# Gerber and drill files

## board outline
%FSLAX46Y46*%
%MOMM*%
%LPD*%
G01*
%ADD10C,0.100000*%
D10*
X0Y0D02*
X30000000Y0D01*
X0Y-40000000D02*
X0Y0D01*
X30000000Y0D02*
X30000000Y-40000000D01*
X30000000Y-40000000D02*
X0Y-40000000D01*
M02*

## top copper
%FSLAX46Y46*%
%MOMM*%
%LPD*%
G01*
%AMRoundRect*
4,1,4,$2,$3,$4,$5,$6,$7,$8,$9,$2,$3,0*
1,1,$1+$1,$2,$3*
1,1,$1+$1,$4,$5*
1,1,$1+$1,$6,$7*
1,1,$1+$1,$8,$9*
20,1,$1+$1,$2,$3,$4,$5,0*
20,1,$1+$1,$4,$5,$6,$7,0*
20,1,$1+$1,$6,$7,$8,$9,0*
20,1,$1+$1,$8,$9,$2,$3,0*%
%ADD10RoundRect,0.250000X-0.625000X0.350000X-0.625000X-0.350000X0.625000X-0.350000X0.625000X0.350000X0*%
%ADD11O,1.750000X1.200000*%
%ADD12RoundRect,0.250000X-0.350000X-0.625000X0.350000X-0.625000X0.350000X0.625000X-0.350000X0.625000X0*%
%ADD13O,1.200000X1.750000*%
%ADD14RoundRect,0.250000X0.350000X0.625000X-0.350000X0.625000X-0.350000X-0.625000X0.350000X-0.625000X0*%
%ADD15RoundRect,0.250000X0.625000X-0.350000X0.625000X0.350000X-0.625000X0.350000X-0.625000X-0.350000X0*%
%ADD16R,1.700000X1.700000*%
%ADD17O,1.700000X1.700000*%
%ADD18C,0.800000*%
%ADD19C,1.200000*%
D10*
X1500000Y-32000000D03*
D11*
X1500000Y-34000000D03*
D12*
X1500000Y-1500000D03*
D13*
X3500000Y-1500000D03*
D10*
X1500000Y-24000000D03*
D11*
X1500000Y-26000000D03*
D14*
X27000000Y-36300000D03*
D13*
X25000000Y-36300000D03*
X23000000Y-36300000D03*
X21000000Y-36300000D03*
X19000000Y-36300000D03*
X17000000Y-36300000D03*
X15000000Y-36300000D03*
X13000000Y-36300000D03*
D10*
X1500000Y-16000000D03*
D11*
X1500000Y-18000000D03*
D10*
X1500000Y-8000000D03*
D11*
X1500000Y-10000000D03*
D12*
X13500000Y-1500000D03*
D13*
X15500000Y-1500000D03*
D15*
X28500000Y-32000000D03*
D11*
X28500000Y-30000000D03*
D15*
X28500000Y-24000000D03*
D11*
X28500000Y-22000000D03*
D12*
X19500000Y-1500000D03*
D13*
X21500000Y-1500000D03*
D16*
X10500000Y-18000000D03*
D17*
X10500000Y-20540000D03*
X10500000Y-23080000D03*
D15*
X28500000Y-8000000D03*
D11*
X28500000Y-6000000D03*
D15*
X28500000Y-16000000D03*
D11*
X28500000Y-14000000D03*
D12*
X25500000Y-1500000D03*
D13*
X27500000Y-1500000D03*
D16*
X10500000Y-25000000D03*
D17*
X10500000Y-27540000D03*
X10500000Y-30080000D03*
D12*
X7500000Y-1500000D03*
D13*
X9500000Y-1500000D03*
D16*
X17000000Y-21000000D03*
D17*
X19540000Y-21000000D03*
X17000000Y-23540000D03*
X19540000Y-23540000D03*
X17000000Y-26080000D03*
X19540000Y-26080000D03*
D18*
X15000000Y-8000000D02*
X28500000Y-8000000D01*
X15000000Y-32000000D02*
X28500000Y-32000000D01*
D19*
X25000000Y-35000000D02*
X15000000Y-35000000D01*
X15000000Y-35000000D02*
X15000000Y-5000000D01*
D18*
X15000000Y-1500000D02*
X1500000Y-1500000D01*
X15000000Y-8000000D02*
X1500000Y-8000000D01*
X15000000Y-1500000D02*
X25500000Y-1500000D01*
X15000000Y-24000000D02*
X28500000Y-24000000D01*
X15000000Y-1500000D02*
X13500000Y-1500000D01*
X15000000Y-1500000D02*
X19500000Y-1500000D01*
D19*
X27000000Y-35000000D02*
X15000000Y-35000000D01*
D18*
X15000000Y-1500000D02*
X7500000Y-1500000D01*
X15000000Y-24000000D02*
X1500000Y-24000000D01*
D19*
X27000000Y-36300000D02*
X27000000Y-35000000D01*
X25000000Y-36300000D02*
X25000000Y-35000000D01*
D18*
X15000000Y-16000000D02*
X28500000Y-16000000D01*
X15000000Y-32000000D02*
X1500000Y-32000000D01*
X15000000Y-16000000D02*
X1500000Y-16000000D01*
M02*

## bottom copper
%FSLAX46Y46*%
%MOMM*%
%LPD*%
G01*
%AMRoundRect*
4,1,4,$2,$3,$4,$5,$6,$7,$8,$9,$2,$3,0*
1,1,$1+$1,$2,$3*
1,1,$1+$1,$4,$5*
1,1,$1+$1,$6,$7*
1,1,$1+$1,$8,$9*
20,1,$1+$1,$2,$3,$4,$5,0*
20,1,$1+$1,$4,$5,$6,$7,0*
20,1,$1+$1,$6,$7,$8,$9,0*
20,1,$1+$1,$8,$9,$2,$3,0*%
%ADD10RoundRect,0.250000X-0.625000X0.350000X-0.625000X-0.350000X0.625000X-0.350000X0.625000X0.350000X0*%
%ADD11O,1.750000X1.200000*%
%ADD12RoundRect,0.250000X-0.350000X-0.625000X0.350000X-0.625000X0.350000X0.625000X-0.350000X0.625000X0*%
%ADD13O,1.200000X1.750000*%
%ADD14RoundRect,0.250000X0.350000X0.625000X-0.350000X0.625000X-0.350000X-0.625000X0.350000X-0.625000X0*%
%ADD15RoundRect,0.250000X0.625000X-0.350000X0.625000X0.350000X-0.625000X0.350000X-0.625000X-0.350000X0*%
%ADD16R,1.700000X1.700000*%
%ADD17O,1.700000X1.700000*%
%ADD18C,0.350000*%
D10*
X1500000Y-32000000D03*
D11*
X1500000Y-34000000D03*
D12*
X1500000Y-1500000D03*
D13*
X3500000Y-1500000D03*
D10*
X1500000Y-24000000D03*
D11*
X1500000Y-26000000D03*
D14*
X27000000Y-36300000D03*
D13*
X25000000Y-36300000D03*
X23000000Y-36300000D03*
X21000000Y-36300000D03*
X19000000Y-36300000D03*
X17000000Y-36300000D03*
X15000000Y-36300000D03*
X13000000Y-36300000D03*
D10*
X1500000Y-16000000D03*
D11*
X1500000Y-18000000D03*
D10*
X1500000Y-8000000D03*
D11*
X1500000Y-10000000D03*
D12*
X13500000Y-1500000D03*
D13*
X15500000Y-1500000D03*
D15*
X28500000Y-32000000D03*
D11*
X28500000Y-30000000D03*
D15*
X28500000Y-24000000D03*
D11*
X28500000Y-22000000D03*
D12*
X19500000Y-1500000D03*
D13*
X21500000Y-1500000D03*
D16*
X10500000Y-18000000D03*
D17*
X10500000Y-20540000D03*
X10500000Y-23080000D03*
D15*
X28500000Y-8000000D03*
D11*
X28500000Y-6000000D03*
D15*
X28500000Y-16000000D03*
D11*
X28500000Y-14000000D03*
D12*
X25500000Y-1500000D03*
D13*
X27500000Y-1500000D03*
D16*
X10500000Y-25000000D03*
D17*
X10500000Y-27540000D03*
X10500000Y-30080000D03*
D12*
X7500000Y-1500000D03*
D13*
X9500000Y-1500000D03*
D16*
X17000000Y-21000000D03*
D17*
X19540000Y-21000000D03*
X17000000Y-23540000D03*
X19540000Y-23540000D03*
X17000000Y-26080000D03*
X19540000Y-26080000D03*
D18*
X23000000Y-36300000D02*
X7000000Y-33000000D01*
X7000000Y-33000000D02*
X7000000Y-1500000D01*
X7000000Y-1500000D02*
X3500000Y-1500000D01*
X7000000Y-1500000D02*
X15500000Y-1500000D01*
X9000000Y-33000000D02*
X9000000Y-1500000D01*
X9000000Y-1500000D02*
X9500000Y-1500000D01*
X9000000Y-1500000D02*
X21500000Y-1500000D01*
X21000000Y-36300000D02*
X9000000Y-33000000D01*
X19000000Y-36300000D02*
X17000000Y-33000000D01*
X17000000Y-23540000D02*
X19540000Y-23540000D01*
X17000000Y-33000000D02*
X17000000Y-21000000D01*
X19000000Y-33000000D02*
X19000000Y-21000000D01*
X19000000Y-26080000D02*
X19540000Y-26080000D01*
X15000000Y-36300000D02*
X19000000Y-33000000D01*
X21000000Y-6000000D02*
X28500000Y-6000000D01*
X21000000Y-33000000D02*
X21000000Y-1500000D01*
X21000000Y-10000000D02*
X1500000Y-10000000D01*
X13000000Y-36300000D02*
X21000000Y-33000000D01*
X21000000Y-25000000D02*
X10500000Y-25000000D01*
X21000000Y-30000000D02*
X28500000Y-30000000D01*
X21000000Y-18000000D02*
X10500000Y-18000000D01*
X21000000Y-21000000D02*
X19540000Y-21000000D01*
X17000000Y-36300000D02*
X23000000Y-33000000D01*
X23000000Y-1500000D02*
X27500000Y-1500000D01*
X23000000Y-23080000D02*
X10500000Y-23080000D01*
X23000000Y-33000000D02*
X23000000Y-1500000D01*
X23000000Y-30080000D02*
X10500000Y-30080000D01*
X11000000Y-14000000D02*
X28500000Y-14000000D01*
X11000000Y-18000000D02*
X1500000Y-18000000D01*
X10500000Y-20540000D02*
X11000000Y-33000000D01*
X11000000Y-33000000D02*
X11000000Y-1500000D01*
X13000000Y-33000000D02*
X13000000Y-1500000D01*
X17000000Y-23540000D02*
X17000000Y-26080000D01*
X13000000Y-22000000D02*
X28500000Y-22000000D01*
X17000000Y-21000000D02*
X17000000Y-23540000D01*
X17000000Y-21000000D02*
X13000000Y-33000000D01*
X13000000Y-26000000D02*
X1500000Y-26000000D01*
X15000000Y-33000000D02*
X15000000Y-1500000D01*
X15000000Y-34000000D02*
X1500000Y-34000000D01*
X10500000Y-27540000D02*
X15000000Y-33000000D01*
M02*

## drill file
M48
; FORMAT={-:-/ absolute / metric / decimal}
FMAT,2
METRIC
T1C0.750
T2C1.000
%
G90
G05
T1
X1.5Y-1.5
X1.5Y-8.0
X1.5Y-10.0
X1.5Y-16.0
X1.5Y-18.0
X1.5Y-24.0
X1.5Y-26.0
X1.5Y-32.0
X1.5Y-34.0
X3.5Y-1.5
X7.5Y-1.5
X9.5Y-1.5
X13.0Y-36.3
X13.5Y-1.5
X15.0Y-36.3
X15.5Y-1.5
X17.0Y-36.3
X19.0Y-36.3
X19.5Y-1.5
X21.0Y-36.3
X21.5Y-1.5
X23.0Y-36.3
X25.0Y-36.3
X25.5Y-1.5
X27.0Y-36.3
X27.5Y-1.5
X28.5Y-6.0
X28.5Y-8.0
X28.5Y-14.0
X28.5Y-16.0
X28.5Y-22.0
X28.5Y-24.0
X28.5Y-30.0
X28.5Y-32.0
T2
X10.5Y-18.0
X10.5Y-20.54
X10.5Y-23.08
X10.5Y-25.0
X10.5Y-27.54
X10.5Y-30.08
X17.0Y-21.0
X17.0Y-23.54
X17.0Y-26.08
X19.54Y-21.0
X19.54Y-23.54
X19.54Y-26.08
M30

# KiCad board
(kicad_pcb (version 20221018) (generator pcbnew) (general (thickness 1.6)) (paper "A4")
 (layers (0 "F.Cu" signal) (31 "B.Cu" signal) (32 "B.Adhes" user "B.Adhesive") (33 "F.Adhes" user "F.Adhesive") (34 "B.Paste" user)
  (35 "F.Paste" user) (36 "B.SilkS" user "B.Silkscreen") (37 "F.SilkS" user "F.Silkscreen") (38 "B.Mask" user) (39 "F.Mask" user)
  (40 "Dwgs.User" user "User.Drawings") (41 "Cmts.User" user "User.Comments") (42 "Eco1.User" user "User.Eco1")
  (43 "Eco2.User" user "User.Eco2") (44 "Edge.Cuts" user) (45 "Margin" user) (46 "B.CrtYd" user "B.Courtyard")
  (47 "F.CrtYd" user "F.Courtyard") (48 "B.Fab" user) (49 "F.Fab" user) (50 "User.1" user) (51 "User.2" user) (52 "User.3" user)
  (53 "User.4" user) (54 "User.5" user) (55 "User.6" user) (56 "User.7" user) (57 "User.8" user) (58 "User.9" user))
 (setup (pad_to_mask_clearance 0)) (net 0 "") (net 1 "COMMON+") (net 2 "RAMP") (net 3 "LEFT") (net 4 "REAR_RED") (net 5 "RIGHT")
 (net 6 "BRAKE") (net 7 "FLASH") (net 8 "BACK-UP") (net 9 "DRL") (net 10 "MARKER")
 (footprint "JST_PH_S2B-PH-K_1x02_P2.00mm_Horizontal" (layer "F.Cu") (at 1.5 32 -90)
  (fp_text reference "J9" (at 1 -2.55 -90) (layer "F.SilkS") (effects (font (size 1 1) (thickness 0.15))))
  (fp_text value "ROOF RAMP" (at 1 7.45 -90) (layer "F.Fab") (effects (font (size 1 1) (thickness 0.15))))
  (pad "1" thru_hole roundrect (at 0 0 270) (size 1.2 1.75) (drill 0.75) (layers "*.Cu" "*.Mask") (roundrect_rratio 0.208333)
   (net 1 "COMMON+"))
  (pad "2" thru_hole oval (at 2 0 270) (size 1.2 1.75) (drill 0.75) (layers "*.Cu" "*.Mask") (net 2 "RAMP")))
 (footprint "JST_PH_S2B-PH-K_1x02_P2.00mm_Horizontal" (layer "F.Cu") (at 1.5 1.5)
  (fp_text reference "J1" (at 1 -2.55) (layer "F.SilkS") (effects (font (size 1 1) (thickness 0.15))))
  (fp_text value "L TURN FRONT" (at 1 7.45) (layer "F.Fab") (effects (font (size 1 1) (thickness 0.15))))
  (pad "1" thru_hole roundrect (at 0 0) (size 1.2 1.75) (drill 0.75) (layers "*.Cu" "*.Mask") (roundrect_rratio 0.208333) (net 1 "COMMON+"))
  (pad "2" thru_hole oval (at 2 0) (size 1.2 1.75) (drill 0.75) (layers "*.Cu" "*.Mask") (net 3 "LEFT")))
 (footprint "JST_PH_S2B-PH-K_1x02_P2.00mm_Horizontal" (layer "F.Cu") (at 1.5 24 -90)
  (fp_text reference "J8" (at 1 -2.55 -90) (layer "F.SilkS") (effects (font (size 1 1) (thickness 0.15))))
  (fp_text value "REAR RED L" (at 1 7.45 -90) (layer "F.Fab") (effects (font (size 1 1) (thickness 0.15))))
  (pad "1" thru_hole roundrect (at 0 0 270) (size 1.2 1.75) (drill 0.75) (layers "*.Cu" "*.Mask") (roundrect_rratio 0.208333)
   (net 1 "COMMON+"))
  (pad "2" thru_hole oval (at 2 0 270) (size 1.2 1.75) (drill 0.75) (layers "*.Cu" "*.Mask") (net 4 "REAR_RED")))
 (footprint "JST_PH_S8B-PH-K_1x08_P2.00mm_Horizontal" (layer "F.Cu") (at 27 36.3 180)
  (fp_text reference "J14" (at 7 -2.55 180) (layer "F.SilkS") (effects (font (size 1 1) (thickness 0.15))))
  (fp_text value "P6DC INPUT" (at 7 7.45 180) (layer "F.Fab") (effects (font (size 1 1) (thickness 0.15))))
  (pad "1" thru_hole roundrect (at 0 0 180) (size 1.2 1.75) (drill 0.75) (layers "*.Cu" "*.Mask") (roundrect_rratio 0.208333)
   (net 1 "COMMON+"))
  (pad "2" thru_hole oval (at 2 0 180) (size 1.2 1.75) (drill 0.75) (layers "*.Cu" "*.Mask") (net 1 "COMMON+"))
  (pad "3" thru_hole oval (at 4 0 180) (size 1.2 1.75) (drill 0.75) (layers "*.Cu" "*.Mask") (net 3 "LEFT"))
  (pad "4" thru_hole oval (at 6 0 180) (size 1.2 1.75) (drill 0.75) (layers "*.Cu" "*.Mask") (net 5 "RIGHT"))
  (pad "5" thru_hole oval (at 8 0 180) (size 1.2 1.75) (drill 0.75) (layers "*.Cu" "*.Mask") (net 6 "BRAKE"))
  (pad "6" thru_hole oval (at 10 0 180) (size 1.2 1.75) (drill 0.75) (layers "*.Cu" "*.Mask") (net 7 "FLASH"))
  (pad "7" thru_hole oval (at 12 0 180) (size 1.2 1.75) (drill 0.75) (layers "*.Cu" "*.Mask") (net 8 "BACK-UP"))
  (pad "8" thru_hole oval (at 14 0 180) (size 1.2 1.75) (drill 0.75) (layers "*.Cu" "*.Mask") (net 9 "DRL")))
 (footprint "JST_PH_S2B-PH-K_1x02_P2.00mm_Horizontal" (layer "F.Cu") (at 1.5 16 -90)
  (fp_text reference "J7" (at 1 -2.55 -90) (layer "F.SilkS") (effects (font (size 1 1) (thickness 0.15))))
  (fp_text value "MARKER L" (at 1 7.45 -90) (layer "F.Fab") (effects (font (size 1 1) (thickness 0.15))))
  (pad "1" thru_hole roundrect (at 0 0 270) (size 1.2 1.75) (drill 0.75) (layers "*.Cu" "*.Mask") (roundrect_rratio 0.208333)
   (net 1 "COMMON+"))
  (pad "2" thru_hole oval (at 2 0 270) (size 1.2 1.75) (drill 0.75) (layers "*.Cu" "*.Mask") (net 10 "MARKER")))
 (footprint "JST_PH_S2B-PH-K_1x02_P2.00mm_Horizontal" (layer "F.Cu") (at 1.5 8 -90)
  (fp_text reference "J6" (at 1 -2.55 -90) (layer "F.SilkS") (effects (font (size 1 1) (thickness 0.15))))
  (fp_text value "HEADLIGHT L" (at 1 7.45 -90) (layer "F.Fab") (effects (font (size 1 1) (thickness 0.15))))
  (pad "1" thru_hole roundrect (at 0 0 270) (size 1.2 1.75) (drill 0.75) (layers "*.Cu" "*.Mask") (roundrect_rratio 0.208333)
   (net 1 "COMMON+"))
  (pad "2" thru_hole oval (at 2 0 270) (size 1.2 1.75) (drill 0.75) (layers "*.Cu" "*.Mask") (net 9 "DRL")))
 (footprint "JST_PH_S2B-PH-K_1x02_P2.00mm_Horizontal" (layer "F.Cu") (at 13.5 1.5)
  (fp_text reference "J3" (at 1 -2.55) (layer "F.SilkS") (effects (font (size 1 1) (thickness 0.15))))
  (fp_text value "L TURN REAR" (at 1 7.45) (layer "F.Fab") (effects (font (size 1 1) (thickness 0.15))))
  (pad "1" thru_hole roundrect (at 0 0) (size 1.2 1.75) (drill 0.75) (layers "*.Cu" "*.Mask") (roundrect_rratio 0.208333) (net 1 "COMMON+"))
  (pad "2" thru_hole oval (at 2 0) (size 1.2 1.75) (drill 0.75) (layers "*.Cu" "*.Mask") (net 3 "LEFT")))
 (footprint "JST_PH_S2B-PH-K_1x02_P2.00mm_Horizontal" (layer "F.Cu") (at 28.5 32 90)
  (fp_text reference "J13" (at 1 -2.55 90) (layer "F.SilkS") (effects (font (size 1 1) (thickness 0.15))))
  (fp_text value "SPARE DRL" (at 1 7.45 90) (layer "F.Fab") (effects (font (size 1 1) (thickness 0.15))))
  (pad "1" thru_hole roundrect (at 0 0 90) (size 1.2 1.75) (drill 0.75) (layers "*.Cu" "*.Mask") (roundrect_rratio 0.208333)
   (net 1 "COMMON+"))
  (pad "2" thru_hole oval (at 2 0 90) (size 1.2 1.75) (drill 0.75) (layers "*.Cu" "*.Mask") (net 9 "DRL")))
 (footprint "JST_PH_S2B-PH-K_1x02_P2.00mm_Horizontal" (layer "F.Cu") (at 28.5 24 90)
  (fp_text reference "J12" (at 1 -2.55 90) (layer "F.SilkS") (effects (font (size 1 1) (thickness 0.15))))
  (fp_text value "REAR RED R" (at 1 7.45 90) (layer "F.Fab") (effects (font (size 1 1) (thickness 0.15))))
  (pad "1" thru_hole roundrect (at 0 0 90) (size 1.2 1.75) (drill 0.75) (layers "*.Cu" "*.Mask") (roundrect_rratio 0.208333)
   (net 1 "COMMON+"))
  (pad "2" thru_hole oval (at 2 0 90) (size 1.2 1.75) (drill 0.75) (layers "*.Cu" "*.Mask") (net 4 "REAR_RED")))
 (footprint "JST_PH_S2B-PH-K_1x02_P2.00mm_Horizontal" (layer "F.Cu") (at 19.5 1.5)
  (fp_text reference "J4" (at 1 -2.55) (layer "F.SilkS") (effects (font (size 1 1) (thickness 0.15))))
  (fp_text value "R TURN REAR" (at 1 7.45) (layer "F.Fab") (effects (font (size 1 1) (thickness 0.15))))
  (pad "1" thru_hole roundrect (at 0 0) (size 1.2 1.75) (drill 0.75) (layers "*.Cu" "*.Mask") (roundrect_rratio 0.208333) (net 1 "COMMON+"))
  (pad "2" thru_hole oval (at 2 0) (size 1.2 1.75) (drill 0.75) (layers "*.Cu" "*.Mask") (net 5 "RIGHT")))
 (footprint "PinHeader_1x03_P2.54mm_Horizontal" (layer "F.Cu") (at 10.5 18)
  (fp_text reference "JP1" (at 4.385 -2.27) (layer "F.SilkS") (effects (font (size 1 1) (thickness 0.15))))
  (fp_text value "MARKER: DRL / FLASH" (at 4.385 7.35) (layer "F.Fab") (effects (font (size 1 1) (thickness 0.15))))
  (pad "1" thru_hole rect (at 0 0) (size 1.7 1.7) (drill 1) (layers "*.Cu" "*.Mask") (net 9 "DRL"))
  (pad "2" thru_hole oval (at 0 2.54) (size 1.7 1.7) (drill 1) (layers "*.Cu" "*.Mask") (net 10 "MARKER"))
  (pad "3" thru_hole oval (at 0 5.08) (size 1.7 1.7) (drill 1) (layers "*.Cu" "*.Mask") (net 7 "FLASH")))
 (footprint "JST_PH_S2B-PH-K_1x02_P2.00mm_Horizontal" (layer "F.Cu") (at 28.5 8 90)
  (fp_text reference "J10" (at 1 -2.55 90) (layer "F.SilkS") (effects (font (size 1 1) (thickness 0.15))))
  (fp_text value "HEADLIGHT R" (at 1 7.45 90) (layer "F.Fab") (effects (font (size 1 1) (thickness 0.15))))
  (pad "1" thru_hole roundrect (at 0 0 90) (size 1.2 1.75) (drill 0.75) (layers "*.Cu" "*.Mask") (roundrect_rratio 0.208333)
   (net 1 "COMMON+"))
  (pad "2" thru_hole oval (at 2 0 90) (size 1.2 1.75) (drill 0.75) (layers "*.Cu" "*.Mask") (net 9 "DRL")))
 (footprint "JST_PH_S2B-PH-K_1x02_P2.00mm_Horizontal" (layer "F.Cu") (at 28.5 16 90)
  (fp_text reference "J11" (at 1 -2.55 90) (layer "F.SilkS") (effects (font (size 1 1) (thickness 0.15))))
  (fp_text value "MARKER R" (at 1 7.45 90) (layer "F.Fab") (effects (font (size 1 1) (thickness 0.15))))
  (pad "1" thru_hole roundrect (at 0 0 90) (size 1.2 1.75) (drill 0.75) (layers "*.Cu" "*.Mask") (roundrect_rratio 0.208333)
   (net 1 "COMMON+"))
  (pad "2" thru_hole oval (at 2 0 90) (size 1.2 1.75) (drill 0.75) (layers "*.Cu" "*.Mask") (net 10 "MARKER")))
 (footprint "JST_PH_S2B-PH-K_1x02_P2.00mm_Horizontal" (layer "F.Cu") (at 25.5 1.5)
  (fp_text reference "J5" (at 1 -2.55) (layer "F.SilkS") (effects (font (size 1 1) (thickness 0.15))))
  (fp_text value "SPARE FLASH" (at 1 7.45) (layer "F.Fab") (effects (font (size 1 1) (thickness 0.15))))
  (pad "1" thru_hole roundrect (at 0 0) (size 1.2 1.75) (drill 0.75) (layers "*.Cu" "*.Mask") (roundrect_rratio 0.208333) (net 1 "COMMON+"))
  (pad "2" thru_hole oval (at 2 0) (size 1.2 1.75) (drill 0.75) (layers "*.Cu" "*.Mask") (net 7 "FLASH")))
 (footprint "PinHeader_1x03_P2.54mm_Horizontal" (layer "F.Cu") (at 10.5 25)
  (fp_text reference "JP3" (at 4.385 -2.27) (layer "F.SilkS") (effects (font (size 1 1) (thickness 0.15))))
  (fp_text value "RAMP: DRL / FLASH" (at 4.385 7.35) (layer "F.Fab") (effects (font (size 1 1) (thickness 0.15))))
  (pad "1" thru_hole rect (at 0 0) (size 1.7 1.7) (drill 1) (layers "*.Cu" "*.Mask") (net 9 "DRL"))
  (pad "2" thru_hole oval (at 0 2.54) (size 1.7 1.7) (drill 1) (layers "*.Cu" "*.Mask") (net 2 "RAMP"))
  (pad "3" thru_hole oval (at 0 5.08) (size 1.7 1.7) (drill 1) (layers "*.Cu" "*.Mask") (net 7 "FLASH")))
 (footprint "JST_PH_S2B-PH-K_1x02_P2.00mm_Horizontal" (layer "F.Cu") (at 7.5 1.5)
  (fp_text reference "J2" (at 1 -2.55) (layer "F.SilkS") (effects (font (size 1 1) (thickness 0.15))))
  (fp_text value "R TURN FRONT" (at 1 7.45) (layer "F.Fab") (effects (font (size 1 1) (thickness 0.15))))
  (pad "1" thru_hole roundrect (at 0 0) (size 1.2 1.75) (drill 0.75) (layers "*.Cu" "*.Mask") (roundrect_rratio 0.208333) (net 1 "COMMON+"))
  (pad "2" thru_hole oval (at 2 0) (size 1.2 1.75) (drill 0.75) (layers "*.Cu" "*.Mask") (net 5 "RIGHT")))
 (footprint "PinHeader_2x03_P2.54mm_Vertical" (layer "F.Cu") (at 17 21)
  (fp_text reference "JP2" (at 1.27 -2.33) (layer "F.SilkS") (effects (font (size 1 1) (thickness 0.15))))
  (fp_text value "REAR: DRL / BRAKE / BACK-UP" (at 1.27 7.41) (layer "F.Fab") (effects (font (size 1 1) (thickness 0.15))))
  (pad "1" thru_hole rect (at 0 0) (size 1.7 1.7) (drill 1) (layers "*.Cu" "*.Mask") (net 4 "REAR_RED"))
  (pad "2" thru_hole oval (at 2.54 0) (size 1.7 1.7) (drill 1) (layers "*.Cu" "*.Mask") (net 9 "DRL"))
  (pad "3" thru_hole oval (at 0 2.54) (size 1.7 1.7) (drill 1) (layers "*.Cu" "*.Mask") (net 4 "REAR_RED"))
  (pad "4" thru_hole oval (at 2.54 2.54) (size 1.7 1.7) (drill 1) (layers "*.Cu" "*.Mask") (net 6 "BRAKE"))
  (pad "5" thru_hole oval (at 0 5.08) (size 1.7 1.7) (drill 1) (layers "*.Cu" "*.Mask") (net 4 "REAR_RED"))
  (pad "6" thru_hole oval (at 2.54 5.08) (size 1.7 1.7) (drill 1) (layers "*.Cu" "*.Mask") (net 8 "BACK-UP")))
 (gr_line (start 0 0) (end 30 0) (stroke (width 0.1) (type default)) (layer "Edge.Cuts"))
 (gr_line (start 0 40) (end 0 0) (stroke (width 0.1) (type default)) (layer "Edge.Cuts"))
 (gr_line (start 30 0) (end 30 40) (stroke (width 0.1) (type default)) (layer "Edge.Cuts"))
 (gr_line (start 30 40) (end 0 40) (stroke (width 0.1) (type default)) (layer "Edge.Cuts"))
 (segment (start 15 8) (end 28.5 8) (width 0.8) (layer "F.Cu") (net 1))
 (segment (start 15 32) (end 28.5 32) (width 0.8) (layer "F.Cu") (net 1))
 (segment (start 25 35) (end 15 35) (width 1.2) (layer "F.Cu") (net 1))
 (segment (start 15 35) (end 15 5) (width 1.2) (layer "F.Cu") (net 1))
 (segment (start 15 1.5) (end 1.5 1.5) (width 0.8) (layer "F.Cu") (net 1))
 (segment (start 15 8) (end 1.5 8) (width 0.8) (layer "F.Cu") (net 1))
 (segment (start 15 1.5) (end 25.5 1.5) (width 0.8) (layer "F.Cu") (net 1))
 (segment (start 15 24) (end 28.5 24) (width 0.8) (layer "F.Cu") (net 1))
 (segment (start 15 1.5) (end 13.5 1.5) (width 0.8) (layer "F.Cu") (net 1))
 (segment (start 15 1.5) (end 19.5 1.5) (width 0.8) (layer "F.Cu") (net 1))
 (segment (start 27 35) (end 15 35) (width 1.2) (layer "F.Cu") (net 1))
 (segment (start 15 1.5) (end 7.5 1.5) (width 0.8) (layer "F.Cu") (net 1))
 (segment (start 15 24) (end 1.5 24) (width 0.8) (layer "F.Cu") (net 1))
 (segment (start 27 36.3) (end 27 35) (width 1.2) (layer "F.Cu") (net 1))
 (segment (start 25 36.3) (end 25 35) (width 1.2) (layer "F.Cu") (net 1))
 (segment (start 15 16) (end 28.5 16) (width 0.8) (layer "F.Cu") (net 1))
 (segment (start 15 32) (end 1.5 32) (width 0.8) (layer "F.Cu") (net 1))
 (segment (start 15 16) (end 1.5 16) (width 0.8) (layer "F.Cu") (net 1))
 (segment (start 23 36.3) (end 7 33) (width 0.35) (layer "B.Cu") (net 3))
 (segment (start 7 33) (end 7 1.5) (width 0.35) (layer "B.Cu") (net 3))
 (segment (start 7 1.5) (end 3.5 1.5) (width 0.35) (layer "B.Cu") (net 3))
 (segment (start 7 1.5) (end 15.5 1.5) (width 0.35) (layer "B.Cu") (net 3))
 (segment (start 9 33) (end 9 1.5) (width 0.35) (layer "B.Cu") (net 5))
 (segment (start 9 1.5) (end 9.5 1.5) (width 0.35) (layer "B.Cu") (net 5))
 (segment (start 9 1.5) (end 21.5 1.5) (width 0.35) (layer "B.Cu") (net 5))
 (segment (start 21 36.3) (end 9 33) (width 0.35) (layer "B.Cu") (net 5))
 (segment (start 19 36.3) (end 17 33) (width 0.35) (layer "B.Cu") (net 6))
 (segment (start 17 23.54) (end 19.54 23.54) (width 0.35) (layer "B.Cu") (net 6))
 (segment (start 17 33) (end 17 21) (width 0.35) (layer "B.Cu") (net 6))
 (segment (start 19 33) (end 19 21) (width 0.35) (layer "B.Cu") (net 8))
 (segment (start 19 26.08) (end 19.54 26.08) (width 0.35) (layer "B.Cu") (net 8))
 (segment (start 15 36.3) (end 19 33) (width 0.35) (layer "B.Cu") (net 8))
 (segment (start 21 6) (end 28.5 6) (width 0.35) (layer "B.Cu") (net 9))
 (segment (start 21 33) (end 21 1.5) (width 0.35) (layer "B.Cu") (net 9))
 (segment (start 21 10) (end 1.5 10) (width 0.35) (layer "B.Cu") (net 9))
 (segment (start 13 36.3) (end 21 33) (width 0.35) (layer "B.Cu") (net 9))
 (segment (start 21 25) (end 10.5 25) (width 0.35) (layer "B.Cu") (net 9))
 (segment (start 21 30) (end 28.5 30) (width 0.35) (layer "B.Cu") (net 9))
 (segment (start 21 18) (end 10.5 18) (width 0.35) (layer "B.Cu") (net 9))
 (segment (start 21 21) (end 19.54 21) (width 0.35) (layer "B.Cu") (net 9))
 (segment (start 17 36.3) (end 23 33) (width 0.35) (layer "B.Cu") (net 7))
 (segment (start 23 1.5) (end 27.5 1.5) (width 0.35) (layer "B.Cu") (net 7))
 (segment (start 23 23.08) (end 10.5 23.08) (width 0.35) (layer "B.Cu") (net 7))
 (segment (start 23 33) (end 23 1.5) (width 0.35) (layer "B.Cu") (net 7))
 (segment (start 23 30.08) (end 10.5 30.08) (width 0.35) (layer "B.Cu") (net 7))
 (segment (start 11 14) (end 28.5 14) (width 0.35) (layer "B.Cu") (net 10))
 (segment (start 11 18) (end 1.5 18) (width 0.35) (layer "B.Cu") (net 10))
 (segment (start 10.5 20.54) (end 11 33) (width 0.35) (layer "B.Cu") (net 10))
 (segment (start 11 33) (end 11 1.5) (width 0.35) (layer "B.Cu") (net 10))
 (segment (start 13 33) (end 13 1.5) (width 0.35) (layer "B.Cu") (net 4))
 (segment (start 17 23.54) (end 17 26.08) (width 0.35) (layer "B.Cu") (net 4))
 (segment (start 13 22) (end 28.5 22) (width 0.35) (layer "B.Cu") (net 4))
 (segment (start 17 21) (end 17 23.54) (width 0.35) (layer "B.Cu") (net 4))
 (segment (start 17 21) (end 13 33) (width 0.35) (layer "B.Cu") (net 4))
 (segment (start 13 26) (end 1.5 26) (width 0.35) (layer "B.Cu") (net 4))
 (segment (start 15 33) (end 15 1.5) (width 0.35) (layer "B.Cu") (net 2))
 (segment (start 15 34) (end 1.5 34) (width 0.35) (layer "B.Cu") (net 2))
 (segment (start 10.5 27.54) (end 15 33) (width 0.35) (layer "B.Cu") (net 2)))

